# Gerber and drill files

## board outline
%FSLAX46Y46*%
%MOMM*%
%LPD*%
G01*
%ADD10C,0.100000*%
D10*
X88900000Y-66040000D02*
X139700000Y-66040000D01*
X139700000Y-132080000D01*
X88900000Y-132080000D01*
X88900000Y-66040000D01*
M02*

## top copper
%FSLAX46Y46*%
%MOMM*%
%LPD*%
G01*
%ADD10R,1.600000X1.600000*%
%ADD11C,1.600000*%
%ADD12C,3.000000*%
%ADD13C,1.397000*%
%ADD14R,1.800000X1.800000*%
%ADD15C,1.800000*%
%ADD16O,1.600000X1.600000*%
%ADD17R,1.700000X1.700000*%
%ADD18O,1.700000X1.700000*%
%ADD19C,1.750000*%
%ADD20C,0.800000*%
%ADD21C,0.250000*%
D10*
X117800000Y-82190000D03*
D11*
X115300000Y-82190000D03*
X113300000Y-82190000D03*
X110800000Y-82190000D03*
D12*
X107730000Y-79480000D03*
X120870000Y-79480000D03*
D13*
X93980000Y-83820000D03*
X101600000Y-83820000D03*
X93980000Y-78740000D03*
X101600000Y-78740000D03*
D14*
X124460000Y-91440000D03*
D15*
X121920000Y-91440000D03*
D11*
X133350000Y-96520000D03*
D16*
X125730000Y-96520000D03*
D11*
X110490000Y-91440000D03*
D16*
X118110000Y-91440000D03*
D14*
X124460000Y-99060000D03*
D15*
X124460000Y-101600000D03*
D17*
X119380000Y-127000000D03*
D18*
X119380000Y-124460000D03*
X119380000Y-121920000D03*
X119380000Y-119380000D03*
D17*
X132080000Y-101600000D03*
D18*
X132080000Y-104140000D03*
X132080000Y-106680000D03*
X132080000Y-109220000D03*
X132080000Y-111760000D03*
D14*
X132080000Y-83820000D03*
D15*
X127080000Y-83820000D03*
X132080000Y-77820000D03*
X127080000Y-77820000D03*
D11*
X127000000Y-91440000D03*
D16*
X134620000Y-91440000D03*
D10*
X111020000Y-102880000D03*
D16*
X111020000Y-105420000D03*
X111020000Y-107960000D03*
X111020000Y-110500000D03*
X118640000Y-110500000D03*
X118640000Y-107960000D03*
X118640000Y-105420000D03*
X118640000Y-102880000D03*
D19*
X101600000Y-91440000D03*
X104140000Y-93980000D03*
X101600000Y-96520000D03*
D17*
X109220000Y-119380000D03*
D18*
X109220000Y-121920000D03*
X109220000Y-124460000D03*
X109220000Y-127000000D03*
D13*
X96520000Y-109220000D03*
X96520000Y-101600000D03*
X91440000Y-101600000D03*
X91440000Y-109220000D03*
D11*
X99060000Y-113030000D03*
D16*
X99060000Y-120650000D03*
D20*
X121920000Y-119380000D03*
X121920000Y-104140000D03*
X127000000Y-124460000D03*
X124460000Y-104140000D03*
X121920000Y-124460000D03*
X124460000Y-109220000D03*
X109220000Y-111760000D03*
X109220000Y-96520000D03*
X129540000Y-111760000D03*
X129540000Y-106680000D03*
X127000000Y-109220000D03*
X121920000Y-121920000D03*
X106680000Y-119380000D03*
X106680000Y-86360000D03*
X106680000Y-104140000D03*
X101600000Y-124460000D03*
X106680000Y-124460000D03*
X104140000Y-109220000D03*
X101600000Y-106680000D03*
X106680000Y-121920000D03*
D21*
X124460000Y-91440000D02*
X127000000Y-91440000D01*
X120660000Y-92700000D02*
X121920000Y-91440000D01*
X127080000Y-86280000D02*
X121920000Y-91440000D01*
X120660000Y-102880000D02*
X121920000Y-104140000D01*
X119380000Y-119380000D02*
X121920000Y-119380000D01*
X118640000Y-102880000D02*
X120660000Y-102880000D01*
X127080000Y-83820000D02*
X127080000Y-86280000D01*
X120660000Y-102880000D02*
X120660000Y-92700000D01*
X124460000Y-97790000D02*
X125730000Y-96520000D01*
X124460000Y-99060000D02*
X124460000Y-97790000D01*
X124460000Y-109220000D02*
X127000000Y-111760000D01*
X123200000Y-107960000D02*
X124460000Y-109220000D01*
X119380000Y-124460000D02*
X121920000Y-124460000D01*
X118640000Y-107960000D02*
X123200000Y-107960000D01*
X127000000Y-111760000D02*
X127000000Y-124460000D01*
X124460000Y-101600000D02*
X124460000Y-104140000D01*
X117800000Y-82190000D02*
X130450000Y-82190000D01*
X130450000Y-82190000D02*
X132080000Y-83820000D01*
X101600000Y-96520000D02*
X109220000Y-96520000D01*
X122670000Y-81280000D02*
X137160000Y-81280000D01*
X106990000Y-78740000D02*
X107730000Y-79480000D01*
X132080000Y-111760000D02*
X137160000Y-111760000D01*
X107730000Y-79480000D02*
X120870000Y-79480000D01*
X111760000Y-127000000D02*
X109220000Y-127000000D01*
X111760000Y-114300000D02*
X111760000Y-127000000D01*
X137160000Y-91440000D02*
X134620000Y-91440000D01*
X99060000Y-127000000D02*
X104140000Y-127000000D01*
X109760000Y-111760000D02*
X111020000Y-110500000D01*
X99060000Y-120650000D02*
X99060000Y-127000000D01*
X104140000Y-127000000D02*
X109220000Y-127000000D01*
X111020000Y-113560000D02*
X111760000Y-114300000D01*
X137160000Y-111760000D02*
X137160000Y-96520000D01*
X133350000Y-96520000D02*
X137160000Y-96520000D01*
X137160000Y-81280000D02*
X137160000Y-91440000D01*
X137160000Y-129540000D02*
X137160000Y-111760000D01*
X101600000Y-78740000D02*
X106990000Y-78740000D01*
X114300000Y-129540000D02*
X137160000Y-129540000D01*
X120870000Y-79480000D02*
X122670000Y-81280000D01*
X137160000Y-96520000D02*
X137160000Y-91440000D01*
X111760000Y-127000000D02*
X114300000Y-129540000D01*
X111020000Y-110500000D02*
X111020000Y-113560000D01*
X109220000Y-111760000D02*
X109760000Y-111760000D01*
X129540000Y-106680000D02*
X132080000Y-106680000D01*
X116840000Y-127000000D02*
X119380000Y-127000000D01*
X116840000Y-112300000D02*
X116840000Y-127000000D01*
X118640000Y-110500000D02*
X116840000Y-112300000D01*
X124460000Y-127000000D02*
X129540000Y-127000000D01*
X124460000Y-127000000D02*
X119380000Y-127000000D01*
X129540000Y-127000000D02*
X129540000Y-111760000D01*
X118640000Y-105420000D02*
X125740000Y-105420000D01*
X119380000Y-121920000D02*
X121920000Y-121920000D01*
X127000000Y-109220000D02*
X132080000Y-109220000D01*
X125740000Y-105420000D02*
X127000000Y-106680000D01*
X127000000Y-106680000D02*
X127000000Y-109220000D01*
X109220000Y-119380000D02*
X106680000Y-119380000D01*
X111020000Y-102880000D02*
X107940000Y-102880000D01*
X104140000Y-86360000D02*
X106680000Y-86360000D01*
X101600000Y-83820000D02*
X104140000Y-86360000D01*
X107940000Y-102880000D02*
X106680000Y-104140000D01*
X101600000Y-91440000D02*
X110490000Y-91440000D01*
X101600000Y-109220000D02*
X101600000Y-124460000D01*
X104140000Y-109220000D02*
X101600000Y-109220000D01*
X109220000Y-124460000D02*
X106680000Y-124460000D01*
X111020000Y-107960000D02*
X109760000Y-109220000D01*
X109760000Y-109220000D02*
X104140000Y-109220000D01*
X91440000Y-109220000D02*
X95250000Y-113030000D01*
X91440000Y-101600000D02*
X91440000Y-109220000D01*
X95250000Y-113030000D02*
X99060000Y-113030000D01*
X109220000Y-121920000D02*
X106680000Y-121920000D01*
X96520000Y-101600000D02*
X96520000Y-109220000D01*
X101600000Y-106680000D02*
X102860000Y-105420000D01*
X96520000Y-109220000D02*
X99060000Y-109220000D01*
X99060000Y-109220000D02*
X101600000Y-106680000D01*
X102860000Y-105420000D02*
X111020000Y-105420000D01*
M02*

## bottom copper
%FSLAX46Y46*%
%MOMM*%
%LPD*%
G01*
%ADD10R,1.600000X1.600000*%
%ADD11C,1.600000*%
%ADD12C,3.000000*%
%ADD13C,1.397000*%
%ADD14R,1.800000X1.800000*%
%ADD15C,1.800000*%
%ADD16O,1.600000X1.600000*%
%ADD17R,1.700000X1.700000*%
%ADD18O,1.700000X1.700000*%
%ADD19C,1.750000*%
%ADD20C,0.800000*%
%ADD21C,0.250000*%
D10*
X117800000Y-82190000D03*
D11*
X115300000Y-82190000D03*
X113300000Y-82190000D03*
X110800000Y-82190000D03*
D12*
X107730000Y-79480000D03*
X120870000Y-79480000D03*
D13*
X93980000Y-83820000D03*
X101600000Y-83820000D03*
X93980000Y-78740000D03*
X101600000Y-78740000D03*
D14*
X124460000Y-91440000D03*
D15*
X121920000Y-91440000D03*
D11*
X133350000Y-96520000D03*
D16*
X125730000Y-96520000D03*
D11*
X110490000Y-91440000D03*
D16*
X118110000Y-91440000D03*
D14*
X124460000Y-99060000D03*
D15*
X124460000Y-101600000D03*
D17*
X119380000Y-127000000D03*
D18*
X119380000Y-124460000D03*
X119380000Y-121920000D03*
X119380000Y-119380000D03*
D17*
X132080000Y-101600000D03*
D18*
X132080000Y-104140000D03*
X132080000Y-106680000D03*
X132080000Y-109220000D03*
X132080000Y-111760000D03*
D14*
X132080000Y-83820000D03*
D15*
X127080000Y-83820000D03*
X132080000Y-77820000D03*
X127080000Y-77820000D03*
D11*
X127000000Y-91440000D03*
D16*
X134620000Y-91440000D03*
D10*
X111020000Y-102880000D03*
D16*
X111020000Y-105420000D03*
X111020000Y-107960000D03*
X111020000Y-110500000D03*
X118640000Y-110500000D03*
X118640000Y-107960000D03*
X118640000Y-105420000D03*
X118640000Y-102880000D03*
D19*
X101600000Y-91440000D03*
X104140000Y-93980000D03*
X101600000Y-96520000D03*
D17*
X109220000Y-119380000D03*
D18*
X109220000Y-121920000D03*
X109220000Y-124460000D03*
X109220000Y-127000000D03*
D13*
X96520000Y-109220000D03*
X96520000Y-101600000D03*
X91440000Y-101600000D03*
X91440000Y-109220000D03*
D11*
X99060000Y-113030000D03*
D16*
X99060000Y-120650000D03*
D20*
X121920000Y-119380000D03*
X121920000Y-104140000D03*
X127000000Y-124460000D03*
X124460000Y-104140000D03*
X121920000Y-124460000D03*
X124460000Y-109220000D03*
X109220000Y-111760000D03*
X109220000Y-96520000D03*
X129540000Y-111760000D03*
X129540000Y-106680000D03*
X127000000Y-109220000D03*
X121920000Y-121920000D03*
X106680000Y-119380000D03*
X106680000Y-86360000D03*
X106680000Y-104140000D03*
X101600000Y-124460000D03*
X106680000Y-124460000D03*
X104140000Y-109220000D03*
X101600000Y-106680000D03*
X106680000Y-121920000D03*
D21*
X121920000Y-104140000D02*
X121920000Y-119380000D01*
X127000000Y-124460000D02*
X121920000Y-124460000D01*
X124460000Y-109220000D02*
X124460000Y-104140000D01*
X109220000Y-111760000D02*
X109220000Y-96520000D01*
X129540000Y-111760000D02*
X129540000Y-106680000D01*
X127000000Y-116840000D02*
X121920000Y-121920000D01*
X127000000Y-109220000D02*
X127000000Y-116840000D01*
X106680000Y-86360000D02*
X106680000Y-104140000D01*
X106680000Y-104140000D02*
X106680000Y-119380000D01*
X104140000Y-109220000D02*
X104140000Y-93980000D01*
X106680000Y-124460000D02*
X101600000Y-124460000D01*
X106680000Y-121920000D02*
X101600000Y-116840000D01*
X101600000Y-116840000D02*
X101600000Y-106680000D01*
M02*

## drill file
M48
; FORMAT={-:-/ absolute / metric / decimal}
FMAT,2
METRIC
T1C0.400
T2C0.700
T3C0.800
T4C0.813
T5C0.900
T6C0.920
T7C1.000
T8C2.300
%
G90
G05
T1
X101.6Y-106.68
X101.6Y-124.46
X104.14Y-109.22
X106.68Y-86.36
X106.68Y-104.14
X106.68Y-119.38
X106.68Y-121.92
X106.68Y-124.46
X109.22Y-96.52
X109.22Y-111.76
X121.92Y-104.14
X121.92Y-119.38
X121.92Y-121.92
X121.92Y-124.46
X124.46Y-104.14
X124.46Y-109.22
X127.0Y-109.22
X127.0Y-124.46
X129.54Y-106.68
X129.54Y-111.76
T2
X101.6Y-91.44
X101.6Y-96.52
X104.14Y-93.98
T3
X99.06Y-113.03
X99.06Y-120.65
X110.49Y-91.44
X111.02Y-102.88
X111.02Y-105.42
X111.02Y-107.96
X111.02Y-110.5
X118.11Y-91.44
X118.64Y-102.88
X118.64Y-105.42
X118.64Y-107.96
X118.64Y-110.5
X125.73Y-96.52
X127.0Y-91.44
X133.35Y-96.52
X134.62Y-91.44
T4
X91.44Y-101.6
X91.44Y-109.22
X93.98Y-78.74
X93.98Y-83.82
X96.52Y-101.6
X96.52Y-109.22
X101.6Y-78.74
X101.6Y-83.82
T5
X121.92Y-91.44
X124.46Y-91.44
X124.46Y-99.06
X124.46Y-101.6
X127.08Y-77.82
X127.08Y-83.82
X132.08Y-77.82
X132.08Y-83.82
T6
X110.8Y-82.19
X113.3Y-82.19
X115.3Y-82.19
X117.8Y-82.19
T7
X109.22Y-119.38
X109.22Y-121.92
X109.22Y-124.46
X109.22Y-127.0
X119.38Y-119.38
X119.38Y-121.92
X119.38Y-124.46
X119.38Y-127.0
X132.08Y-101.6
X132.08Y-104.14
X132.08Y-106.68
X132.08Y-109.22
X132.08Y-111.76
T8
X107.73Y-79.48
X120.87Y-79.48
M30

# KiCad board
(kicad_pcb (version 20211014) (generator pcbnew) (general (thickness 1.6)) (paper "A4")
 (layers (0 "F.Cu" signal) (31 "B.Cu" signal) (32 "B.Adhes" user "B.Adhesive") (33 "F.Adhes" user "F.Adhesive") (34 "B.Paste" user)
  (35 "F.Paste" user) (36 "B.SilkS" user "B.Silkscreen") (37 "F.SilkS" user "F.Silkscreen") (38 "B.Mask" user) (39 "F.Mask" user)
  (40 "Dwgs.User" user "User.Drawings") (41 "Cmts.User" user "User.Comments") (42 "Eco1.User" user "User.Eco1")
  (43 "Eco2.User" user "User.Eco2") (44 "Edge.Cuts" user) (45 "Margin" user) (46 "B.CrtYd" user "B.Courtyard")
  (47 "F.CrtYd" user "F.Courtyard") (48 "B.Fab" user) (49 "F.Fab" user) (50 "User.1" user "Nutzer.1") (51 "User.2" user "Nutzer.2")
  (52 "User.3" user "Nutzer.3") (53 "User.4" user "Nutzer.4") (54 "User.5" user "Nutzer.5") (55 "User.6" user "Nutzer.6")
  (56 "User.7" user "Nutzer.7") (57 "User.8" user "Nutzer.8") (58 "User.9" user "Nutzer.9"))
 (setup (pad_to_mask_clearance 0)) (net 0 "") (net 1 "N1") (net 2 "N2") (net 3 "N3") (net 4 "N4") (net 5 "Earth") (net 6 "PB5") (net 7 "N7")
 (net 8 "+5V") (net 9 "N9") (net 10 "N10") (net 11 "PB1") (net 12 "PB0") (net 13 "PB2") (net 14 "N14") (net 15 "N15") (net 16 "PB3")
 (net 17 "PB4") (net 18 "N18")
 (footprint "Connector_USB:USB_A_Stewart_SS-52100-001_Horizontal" (layer "F.Cu") (at 117.8 82.19 180)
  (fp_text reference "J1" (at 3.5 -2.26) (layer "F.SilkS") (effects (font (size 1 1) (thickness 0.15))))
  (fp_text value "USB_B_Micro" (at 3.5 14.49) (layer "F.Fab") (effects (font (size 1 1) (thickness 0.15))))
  (pad "1" thru_hole rect (at 0 0 180) (size 1.6 1.6) (drill 0.92) (layers *.Cu *.Mask) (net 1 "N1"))
  (pad "2" thru_hole circle (at 2.5 0 180) (size 1.6 1.6) (drill 0.92) (layers *.Cu *.Mask) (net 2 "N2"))
  (pad "3" thru_hole circle (at 4.5 0 180) (size 1.6 1.6) (drill 0.92) (layers *.Cu *.Mask) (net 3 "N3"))
  (pad "4" thru_hole circle (at 7 0 180) (size 1.6 1.6) (drill 0.92) (layers *.Cu *.Mask) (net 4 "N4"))
  (pad "5" thru_hole circle (at 10.07 2.71 180) (size 3 3) (drill 2.3) (layers *.Cu *.Mask) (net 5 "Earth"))
  (pad "5" thru_hole circle (at -3.07 2.71 180) (size 3 3) (drill 2.3) (layers *.Cu *.Mask) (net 5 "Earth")))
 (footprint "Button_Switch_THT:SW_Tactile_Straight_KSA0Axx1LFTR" (layer "F.Cu") (at 101.6 83.82 180)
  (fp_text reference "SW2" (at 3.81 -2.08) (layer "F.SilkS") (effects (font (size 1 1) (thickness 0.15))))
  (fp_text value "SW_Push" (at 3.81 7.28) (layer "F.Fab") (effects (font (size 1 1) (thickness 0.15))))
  (pad "1" thru_hole circle (at 7.62 0 180) (size 1.397 1.397) (drill 0.8128) (layers *.Cu *.Mask) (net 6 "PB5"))
  (pad "1" thru_hole circle (at 0 0 180) (size 1.397 1.397) (drill 0.8128) (layers *.Cu *.Mask) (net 6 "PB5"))
  (pad "2" thru_hole circle (at 7.62 5.08 180) (size 1.397 1.397) (drill 0.8128) (layers *.Cu *.Mask) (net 5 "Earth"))
  (pad "2" thru_hole circle (at 0 5.08 180) (size 1.397 1.397) (drill 0.8128) (layers *.Cu *.Mask) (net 5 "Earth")))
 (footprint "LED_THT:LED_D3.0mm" (layer "F.Cu") (at 124.46 91.44 180)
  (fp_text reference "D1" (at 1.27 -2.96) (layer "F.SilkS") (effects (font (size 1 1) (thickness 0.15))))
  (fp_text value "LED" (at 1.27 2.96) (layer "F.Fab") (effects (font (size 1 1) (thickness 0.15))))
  (pad "1" thru_hole rect (at 0 0 180) (size 1.8 1.8) (drill 0.9) (layers *.Cu *.Mask) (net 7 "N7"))
  (pad "2" thru_hole circle (at 2.54 0 180) (size 1.8 1.8) (drill 0.9) (layers *.Cu *.Mask) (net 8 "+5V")))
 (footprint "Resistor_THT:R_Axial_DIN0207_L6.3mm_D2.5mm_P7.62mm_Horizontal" (layer "F.Cu") (at 133.35 96.52 180)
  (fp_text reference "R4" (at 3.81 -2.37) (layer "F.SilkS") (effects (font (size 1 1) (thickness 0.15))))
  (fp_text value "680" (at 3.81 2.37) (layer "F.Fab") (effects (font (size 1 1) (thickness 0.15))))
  (pad "1" thru_hole circle (at 0 0 180) (size 1.6 1.6) (drill 0.8) (layers *.Cu *.Mask) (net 5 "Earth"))
  (pad "2" thru_hole oval (at 7.62 0 180) (size 1.6 1.6) (drill 0.8) (layers *.Cu *.Mask) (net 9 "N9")))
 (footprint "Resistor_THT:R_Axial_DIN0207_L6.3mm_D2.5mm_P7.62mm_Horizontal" (layer "F.Cu") (at 110.49 91.44)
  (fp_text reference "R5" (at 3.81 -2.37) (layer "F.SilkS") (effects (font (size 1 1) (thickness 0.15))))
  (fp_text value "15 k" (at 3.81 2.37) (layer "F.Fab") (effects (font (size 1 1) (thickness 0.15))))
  (pad "1" thru_hole circle (at 0 0) (size 1.6 1.6) (drill 0.8) (layers *.Cu *.Mask) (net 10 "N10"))
  (pad "2" thru_hole oval (at 7.62 0) (size 1.6 1.6) (drill 0.8) (layers *.Cu *.Mask) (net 8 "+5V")))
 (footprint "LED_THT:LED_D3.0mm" (layer "F.Cu") (at 124.46 99.06 -90)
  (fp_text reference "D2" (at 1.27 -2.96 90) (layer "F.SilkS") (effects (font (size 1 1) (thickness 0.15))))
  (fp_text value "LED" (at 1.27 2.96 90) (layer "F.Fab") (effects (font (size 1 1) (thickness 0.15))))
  (pad "1" thru_hole rect (at 0 0 270) (size 1.8 1.8) (drill 0.9) (layers *.Cu *.Mask) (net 9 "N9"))
  (pad "2" thru_hole circle (at 2.54 0 270) (size 1.8 1.8) (drill 0.9) (layers *.Cu *.Mask) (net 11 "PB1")))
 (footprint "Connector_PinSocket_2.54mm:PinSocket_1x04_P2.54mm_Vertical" (layer "F.Cu") (at 119.38 127 180)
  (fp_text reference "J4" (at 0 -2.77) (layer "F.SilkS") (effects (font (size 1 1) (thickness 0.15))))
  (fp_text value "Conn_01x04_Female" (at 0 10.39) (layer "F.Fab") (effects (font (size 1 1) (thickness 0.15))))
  (pad "1" thru_hole rect (at 0 0 180) (size 1.7 1.7) (drill 1) (layers *.Cu *.Mask) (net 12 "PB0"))
  (pad "2" thru_hole oval (at 0 2.54 180) (size 1.7 1.7) (drill 1) (layers *.Cu *.Mask) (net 11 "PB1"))
  (pad "3" thru_hole oval (at 0 5.08 180) (size 1.7 1.7) (drill 1) (layers *.Cu *.Mask) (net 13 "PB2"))
  (pad "4" thru_hole oval (at 0 7.62 180) (size 1.7 1.7) (drill 1) (layers *.Cu *.Mask) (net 8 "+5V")))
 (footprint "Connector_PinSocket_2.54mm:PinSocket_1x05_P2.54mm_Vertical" (layer "F.Cu") (at 132.08 101.6)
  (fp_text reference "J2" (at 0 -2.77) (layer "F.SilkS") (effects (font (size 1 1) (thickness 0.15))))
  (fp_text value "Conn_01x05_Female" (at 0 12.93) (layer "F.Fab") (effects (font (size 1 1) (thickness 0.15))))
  (pad "1" thru_hole rect (at 0 0) (size 1.7 1.7) (drill 1) (layers *.Cu *.Mask) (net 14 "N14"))
  (pad "2" thru_hole oval (at 0 2.54) (size 1.7 1.7) (drill 1) (layers *.Cu *.Mask) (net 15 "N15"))
  (pad "3" thru_hole oval (at 0 5.08) (size 1.7 1.7) (drill 1) (layers *.Cu *.Mask) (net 12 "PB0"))
  (pad "4" thru_hole oval (at 0 7.62) (size 1.7 1.7) (drill 1) (layers *.Cu *.Mask) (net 13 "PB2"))
  (pad "5" thru_hole oval (at 0 10.16) (size 1.7 1.7) (drill 1) (layers *.Cu *.Mask) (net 5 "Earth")))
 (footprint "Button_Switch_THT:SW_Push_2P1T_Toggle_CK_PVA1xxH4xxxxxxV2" (layer "F.Cu") (at 132.08 83.82 180)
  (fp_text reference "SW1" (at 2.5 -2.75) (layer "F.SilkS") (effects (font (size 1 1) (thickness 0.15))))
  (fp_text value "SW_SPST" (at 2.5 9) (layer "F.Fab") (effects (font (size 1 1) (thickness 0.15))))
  (pad "1" thru_hole rect (at 0 0 180) (size 1.8 1.8) (drill 0.9) (layers *.Cu *.Mask) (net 1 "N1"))
  (pad "2" thru_hole circle (at 5 0 180) (size 1.8 1.8) (drill 0.9) (layers *.Cu *.Mask) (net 8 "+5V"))
  (pad "3" thru_hole circle (at 0 6 180) (size 1.8 1.8) (drill 0.9) (layers *.Cu *.Mask))
  (pad "4" thru_hole circle (at 5 6 180) (size 1.8 1.8) (drill 0.9) (layers *.Cu *.Mask)))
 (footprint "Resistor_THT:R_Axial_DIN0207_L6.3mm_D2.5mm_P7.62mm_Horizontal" (layer "F.Cu") (at 127 91.44)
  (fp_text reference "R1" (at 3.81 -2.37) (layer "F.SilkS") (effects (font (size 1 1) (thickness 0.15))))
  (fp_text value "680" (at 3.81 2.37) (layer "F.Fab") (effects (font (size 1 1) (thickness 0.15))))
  (pad "1" thru_hole circle (at 0 0) (size 1.6 1.6) (drill 0.8) (layers *.Cu *.Mask) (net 7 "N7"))
  (pad "2" thru_hole oval (at 7.62 0) (size 1.6 1.6) (drill 0.8) (layers *.Cu *.Mask) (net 5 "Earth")))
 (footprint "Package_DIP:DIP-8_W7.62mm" (layer "F.Cu") (at 111.02 102.88)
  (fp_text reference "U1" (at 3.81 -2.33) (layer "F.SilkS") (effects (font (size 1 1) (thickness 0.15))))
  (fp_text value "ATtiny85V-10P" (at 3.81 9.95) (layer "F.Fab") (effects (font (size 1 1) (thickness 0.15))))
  (pad "1" thru_hole rect (at 0 0) (size 1.6 1.6) (drill 0.8) (layers *.Cu *.Mask) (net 6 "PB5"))
  (pad "2" thru_hole oval (at 0 2.54) (size 1.6 1.6) (drill 0.8) (layers *.Cu *.Mask) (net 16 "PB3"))
  (pad "3" thru_hole oval (at 0 5.08) (size 1.6 1.6) (drill 0.8) (layers *.Cu *.Mask) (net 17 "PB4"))
  (pad "4" thru_hole oval (at 0 7.62) (size 1.6 1.6) (drill 0.8) (layers *.Cu *.Mask) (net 5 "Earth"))
  (pad "5" thru_hole oval (at 7.62 7.62) (size 1.6 1.6) (drill 0.8) (layers *.Cu *.Mask) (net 12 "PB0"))
  (pad "6" thru_hole oval (at 7.62 5.08) (size 1.6 1.6) (drill 0.8) (layers *.Cu *.Mask) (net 11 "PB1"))
  (pad "7" thru_hole oval (at 7.62 2.54) (size 1.6 1.6) (drill 0.8) (layers *.Cu *.Mask) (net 13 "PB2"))
  (pad "8" thru_hole oval (at 7.62 0) (size 1.6 1.6) (drill 0.8) (layers *.Cu *.Mask) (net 8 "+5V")))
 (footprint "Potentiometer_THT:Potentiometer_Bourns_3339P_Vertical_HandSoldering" (layer "F.Cu") (at 101.6 91.44 180)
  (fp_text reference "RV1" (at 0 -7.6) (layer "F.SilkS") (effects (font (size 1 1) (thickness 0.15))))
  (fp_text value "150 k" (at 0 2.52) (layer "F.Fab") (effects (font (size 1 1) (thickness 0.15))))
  (pad "1" thru_hole circle (at 0 0 180) (size 1.75 1.75) (drill 0.7) (layers *.Cu *.Mask) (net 10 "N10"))
  (pad "2" thru_hole circle (at -2.54 -2.54 180) (size 1.75 1.75) (drill 0.7) (layers *.Cu *.Mask) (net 17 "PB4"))
  (pad "3" thru_hole circle (at 0 -5.08 180) (size 1.75 1.75) (drill 0.7) (layers *.Cu *.Mask) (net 5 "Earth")))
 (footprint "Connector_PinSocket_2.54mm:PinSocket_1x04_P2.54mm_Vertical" (layer "F.Cu") (at 109.22 119.38)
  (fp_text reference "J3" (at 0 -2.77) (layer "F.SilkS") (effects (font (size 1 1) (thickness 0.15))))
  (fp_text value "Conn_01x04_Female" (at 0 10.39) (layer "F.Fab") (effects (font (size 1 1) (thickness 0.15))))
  (pad "1" thru_hole rect (at 0 0) (size 1.7 1.7) (drill 1) (layers *.Cu *.Mask) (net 6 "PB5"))
  (pad "2" thru_hole oval (at 0 2.54) (size 1.7 1.7) (drill 1) (layers *.Cu *.Mask) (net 16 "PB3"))
  (pad "3" thru_hole oval (at 0 5.08) (size 1.7 1.7) (drill 1) (layers *.Cu *.Mask) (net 17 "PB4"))
  (pad "4" thru_hole oval (at 0 7.62) (size 1.7 1.7) (drill 1) (layers *.Cu *.Mask) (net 5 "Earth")))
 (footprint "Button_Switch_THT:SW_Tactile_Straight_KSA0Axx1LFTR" (layer "F.Cu") (at 96.52 101.6 -90)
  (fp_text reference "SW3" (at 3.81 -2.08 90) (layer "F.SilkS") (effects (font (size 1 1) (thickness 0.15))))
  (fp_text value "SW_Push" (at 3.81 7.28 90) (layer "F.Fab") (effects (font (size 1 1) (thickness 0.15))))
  (pad "1" thru_hole circle (at 7.62 0 270) (size 1.397 1.397) (drill 0.8128) (layers *.Cu *.Mask) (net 16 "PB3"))
  (pad "1" thru_hole circle (at 0 0 270) (size 1.397 1.397) (drill 0.8128) (layers *.Cu *.Mask) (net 16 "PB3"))
  (pad "2" thru_hole circle (at 0 5.08 270) (size 1.397 1.397) (drill 0.8128) (layers *.Cu *.Mask) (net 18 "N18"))
  (pad "2" thru_hole circle (at 7.62 5.08 270) (size 1.397 1.397) (drill 0.8128) (layers *.Cu *.Mask) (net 18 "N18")))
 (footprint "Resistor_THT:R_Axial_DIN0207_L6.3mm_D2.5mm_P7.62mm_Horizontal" (layer "F.Cu") (at 99.06 113.03 -90)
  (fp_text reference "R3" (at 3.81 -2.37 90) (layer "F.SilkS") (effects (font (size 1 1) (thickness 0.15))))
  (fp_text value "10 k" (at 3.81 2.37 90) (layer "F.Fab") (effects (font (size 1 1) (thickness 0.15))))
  (pad "1" thru_hole circle (at 0 0 270) (size 1.6 1.6) (drill 0.8) (layers *.Cu *.Mask) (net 18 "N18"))
  (pad "2" thru_hole oval (at 7.62 0 270) (size 1.6 1.6) (drill 0.8) (layers *.Cu *.Mask) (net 5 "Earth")))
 (gr_rect (start 139.7 132.08) (end 88.9 66.04) (layer "Edge.Cuts") (width 0.1) (fill none))
 (segment (start 124.46 91.44) (end 127 91.44) (width 0.25) (layer "F.Cu") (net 7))
 (segment (start 120.66 92.7) (end 121.92 91.44) (width 0.25) (layer "F.Cu") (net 8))
 (segment (start 127.08 86.28) (end 121.92 91.44) (width 0.25) (layer "F.Cu") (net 8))
 (segment (start 120.66 102.88) (end 121.92 104.14) (width 0.25) (layer "F.Cu") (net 8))
 (segment (start 119.38 119.38) (end 121.92 119.38) (width 0.25) (layer "F.Cu") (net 8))
 (segment (start 118.64 102.88) (end 120.66 102.88) (width 0.25) (layer "F.Cu") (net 8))
 (segment (start 127.08 83.82) (end 127.08 86.28) (width 0.25) (layer "F.Cu") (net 8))
 (segment (start 120.66 102.88) (end 120.66 92.7) (width 0.25) (layer "F.Cu") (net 8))
 (via (at 121.92 119.38) (size 0.8) (drill 0.4) (layers "F.Cu" "B.Cu") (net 8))
 (via (at 121.92 104.14) (size 0.8) (drill 0.4) (layers "F.Cu" "B.Cu") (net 8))
 (segment (start 121.92 104.14) (end 121.92 119.38) (width 0.25) (layer "B.Cu") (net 8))
 (segment (start 124.46 97.79) (end 125.73 96.52) (width 0.25) (layer "F.Cu") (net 9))
 (segment (start 124.46 99.06) (end 124.46 97.79) (width 0.25) (layer "F.Cu") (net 9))
 (segment (start 124.46 109.22) (end 127 111.76) (width 0.25) (layer "F.Cu") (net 11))
 (segment (start 123.2 107.96) (end 124.46 109.22) (width 0.25) (layer "F.Cu") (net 11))
 (segment (start 119.38 124.46) (end 121.92 124.46) (width 0.25) (layer "F.Cu") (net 11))
 (segment (start 118.64 107.96) (end 123.2 107.96) (width 0.25) (layer "F.Cu") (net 11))
 (segment (start 127 111.76) (end 127 124.46) (width 0.25) (layer "F.Cu") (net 11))
 (segment (start 124.46 101.6) (end 124.46 104.14) (width 0.25) (layer "F.Cu") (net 11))
 (via (at 127 124.46) (size 0.8) (drill 0.4) (layers "F.Cu" "B.Cu") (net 11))
 (via (at 124.46 104.14) (size 0.8) (drill 0.4) (layers "F.Cu" "B.Cu") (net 11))
 (via (at 121.92 124.46) (size 0.8) (drill 0.4) (layers "F.Cu" "B.Cu") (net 11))
 (via (at 124.46 109.22) (size 0.8) (drill 0.4) (layers "F.Cu" "B.Cu") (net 11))
 (segment (start 127 124.46) (end 121.92 124.46) (width 0.25) (layer "B.Cu") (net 11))
 (segment (start 124.46 109.22) (end 124.46 104.14) (width 0.25) (layer "B.Cu") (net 11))
 (segment (start 117.8 82.19) (end 130.45 82.19) (width 0.25) (layer "F.Cu") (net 1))
 (segment (start 130.45 82.19) (end 132.08 83.82) (width 0.25) (layer "F.Cu") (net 1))
 (segment (start 101.6 96.52) (end 109.22 96.52) (width 0.25) (layer "F.Cu") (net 5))
 (segment (start 122.67 81.28) (end 137.16 81.28) (width 0.25) (layer "F.Cu") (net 5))
 (segment (start 106.99 78.74) (end 107.73 79.48) (width 0.25) (layer "F.Cu") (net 5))
 (segment (start 132.08 111.76) (end 137.16 111.76) (width 0.25) (layer "F.Cu") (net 5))
 (segment (start 107.73 79.48) (end 120.87 79.48) (width 0.25) (layer "F.Cu") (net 5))
 (segment (start 111.76 127) (end 109.22 127) (width 0.25) (layer "F.Cu") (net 5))
 (segment (start 111.76 114.3) (end 111.76 127) (width 0.25) (layer "F.Cu") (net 5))
 (segment (start 137.16 91.44) (end 134.62 91.44) (width 0.25) (layer "F.Cu") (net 5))
 (segment (start 99.06 127) (end 104.14 127) (width 0.25) (layer "F.Cu") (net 5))
 (segment (start 109.76 111.76) (end 111.02 110.5) (width 0.25) (layer "F.Cu") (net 5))
 (segment (start 99.06 120.65) (end 99.06 127) (width 0.25) (layer "F.Cu") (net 5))
 (segment (start 104.14 127) (end 109.22 127) (width 0.25) (layer "F.Cu") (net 5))
 (segment (start 111.02 113.56) (end 111.76 114.3) (width 0.25) (layer "F.Cu") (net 5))
 (segment (start 137.16 111.76) (end 137.16 96.52) (width 0.25) (layer "F.Cu") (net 5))
 (segment (start 133.35 96.52) (end 137.16 96.52) (width 0.25) (layer "F.Cu") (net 5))
 (segment (start 137.16 81.28) (end 137.16 91.44) (width 0.25) (layer "F.Cu") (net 5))
 (segment (start 137.16 129.54) (end 137.16 111.76) (width 0.25) (layer "F.Cu") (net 5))
 (segment (start 101.6 78.74) (end 106.99 78.74) (width 0.25) (layer "F.Cu") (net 5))
 (segment (start 114.3 129.54) (end 137.16 129.54) (width 0.25) (layer "F.Cu") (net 5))
 (segment (start 120.87 79.48) (end 122.67 81.28) (width 0.25) (layer "F.Cu") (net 5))
 (segment (start 137.16 96.52) (end 137.16 91.44) (width 0.25) (layer "F.Cu") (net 5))
 (segment (start 111.76 127) (end 114.3 129.54) (width 0.25) (layer "F.Cu") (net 5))
 (segment (start 111.02 110.5) (end 111.02 113.56) (width 0.25) (layer "F.Cu") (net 5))
 (segment (start 109.22 111.76) (end 109.76 111.76) (width 0.25) (layer "F.Cu") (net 5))
 (via (at 109.22 111.76) (size 0.8) (drill 0.4) (layers "F.Cu" "B.Cu") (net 5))
 (via (at 109.22 96.52) (size 0.8) (drill 0.4) (layers "F.Cu" "B.Cu") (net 5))
 (segment (start 109.22 111.76) (end 109.22 96.52) (width 0.25) (layer "B.Cu") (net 5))
 (segment (start 129.54 106.68) (end 132.08 106.68) (width 0.25) (layer "F.Cu") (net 12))
 (segment (start 116.84 127) (end 119.38 127) (width 0.25) (layer "F.Cu") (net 12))
 (segment (start 116.84 112.3) (end 116.84 127) (width 0.25) (layer "F.Cu") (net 12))
 (segment (start 118.64 110.5) (end 116.84 112.3) (width 0.25) (layer "F.Cu") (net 12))
 (segment (start 124.46 127) (end 129.54 127) (width 0.25) (layer "F.Cu") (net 12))
 (segment (start 124.46 127) (end 119.38 127) (width 0.25) (layer "F.Cu") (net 12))
 (segment (start 129.54 127) (end 129.54 111.76) (width 0.25) (layer "F.Cu") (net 12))
 (via (at 129.54 111.76) (size 0.8) (drill 0.4) (layers "F.Cu" "B.Cu") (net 12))
 (via (at 129.54 106.68) (size 0.8) (drill 0.4) (layers "F.Cu" "B.Cu") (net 12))
 (segment (start 129.54 111.76) (end 129.54 106.68) (width 0.25) (layer "B.Cu") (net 12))
 (segment (start 118.64 105.42) (end 125.74 105.42) (width 0.25) (layer "F.Cu") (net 13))
 (segment (start 119.38 121.92) (end 121.92 121.92) (width 0.25) (layer "F.Cu") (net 13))
 (segment (start 127 109.22) (end 132.08 109.22) (width 0.25) (layer "F.Cu") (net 13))
 (segment (start 125.74 105.42) (end 127 106.68) (width 0.25) (layer "F.Cu") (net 13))
 (segment (start 127 106.68) (end 127 109.22) (width 0.25) (layer "F.Cu") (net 13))
 (via (at 127 109.22) (size 0.8) (drill 0.4) (layers "F.Cu" "B.Cu") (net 13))
 (via (at 121.92 121.92) (size 0.8) (drill 0.4) (layers "F.Cu" "B.Cu") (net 13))
 (segment (start 127 116.84) (end 121.92 121.92) (width 0.25) (layer "B.Cu") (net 13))
 (segment (start 127 109.22) (end 127 116.84) (width 0.25) (layer "B.Cu") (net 13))
 (segment (start 109.22 119.38) (end 106.68 119.38) (width 0.25) (layer "F.Cu") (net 6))
 (segment (start 111.02 102.88) (end 107.94 102.88) (width 0.25) (layer "F.Cu") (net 6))
 (segment (start 104.14 86.36) (end 106.68 86.36) (width 0.25) (layer "F.Cu") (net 6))
 (segment (start 101.6 83.82) (end 104.14 86.36) (width 0.25) (layer "F.Cu") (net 6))
 (segment (start 107.94 102.88) (end 106.68 104.14) (width 0.25) (layer "F.Cu") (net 6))
 (via (at 106.68 119.38) (size 0.8) (drill 0.4) (layers "F.Cu" "B.Cu") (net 6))
 (via (at 106.68 86.36) (size 0.8) (drill 0.4) (layers "F.Cu" "B.Cu") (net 6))
 (via (at 106.68 104.14) (size 0.8) (drill 0.4) (layers "F.Cu" "B.Cu") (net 6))
 (segment (start 106.68 86.36) (end 106.68 104.14) (width 0.25) (layer "B.Cu") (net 6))
 (segment (start 106.68 104.14) (end 106.68 119.38) (width 0.25) (layer "B.Cu") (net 6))
 (segment (start 101.6 91.44) (end 110.49 91.44) (width 0.25) (layer "F.Cu") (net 10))
 (segment (start 101.6 109.22) (end 101.6 124.46) (width 0.25) (layer "F.Cu") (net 17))
 (segment (start 104.14 109.22) (end 101.6 109.22) (width 0.25) (layer "F.Cu") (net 17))
 (segment (start 109.22 124.46) (end 106.68 124.46) (width 0.25) (layer "F.Cu") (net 17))
 (segment (start 111.02 107.96) (end 109.76 109.22) (width 0.25) (layer "F.Cu") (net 17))
 (segment (start 109.76 109.22) (end 104.14 109.22) (width 0.25) (layer "F.Cu") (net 17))
 (via (at 101.6 124.46) (size 0.8) (drill 0.4) (layers "F.Cu" "B.Cu") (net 17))
 (via (at 106.68 124.46) (size 0.8) (drill 0.4) (layers "F.Cu" "B.Cu") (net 17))
 (via (at 104.14 109.22) (size 0.8) (drill 0.4) (layers "F.Cu" "B.Cu") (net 17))
 (segment (start 104.14 109.22) (end 104.14 93.98) (width 0.25) (layer "B.Cu") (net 17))
 (segment (start 106.68 124.46) (end 101.6 124.46) (width 0.25) (layer "B.Cu") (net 17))
 (segment (start 91.44 109.22) (end 95.25 113.03) (width 0.25) (layer "F.Cu") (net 18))
 (segment (start 91.44 101.6) (end 91.44 109.22) (width 0.25) (layer "F.Cu") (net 18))
 (segment (start 95.25 113.03) (end 99.06 113.03) (width 0.25) (layer "F.Cu") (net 18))
 (segment (start 109.22 121.92) (end 106.68 121.92) (width 0.25) (layer "F.Cu") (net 16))
 (segment (start 96.52 101.6) (end 96.52 109.22) (width 0.25) (layer "F.Cu") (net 16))
 (segment (start 101.6 106.68) (end 102.86 105.42) (width 0.25) (layer "F.Cu") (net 16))
 (segment (start 96.52 109.22) (end 99.06 109.22) (width 0.25) (layer "F.Cu") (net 16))
 (segment (start 99.06 109.22) (end 101.6 106.68) (width 0.25) (layer "F.Cu") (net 16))
 (segment (start 102.86 105.42) (end 111.02 105.42) (width 0.25) (layer "F.Cu") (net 16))
 (via (at 101.6 106.68) (size 0.8) (drill 0.4) (layers "F.Cu" "B.Cu") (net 16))
 (via (at 106.68 121.92) (size 0.8) (drill 0.4) (layers "F.Cu" "B.Cu") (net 16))
 (segment (start 106.68 121.92) (end 101.6 116.84) (width 0.25) (layer "B.Cu") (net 16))
 (segment (start 101.6 116.84) (end 101.6 106.68) (width 0.25) (layer "B.Cu") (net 16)))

